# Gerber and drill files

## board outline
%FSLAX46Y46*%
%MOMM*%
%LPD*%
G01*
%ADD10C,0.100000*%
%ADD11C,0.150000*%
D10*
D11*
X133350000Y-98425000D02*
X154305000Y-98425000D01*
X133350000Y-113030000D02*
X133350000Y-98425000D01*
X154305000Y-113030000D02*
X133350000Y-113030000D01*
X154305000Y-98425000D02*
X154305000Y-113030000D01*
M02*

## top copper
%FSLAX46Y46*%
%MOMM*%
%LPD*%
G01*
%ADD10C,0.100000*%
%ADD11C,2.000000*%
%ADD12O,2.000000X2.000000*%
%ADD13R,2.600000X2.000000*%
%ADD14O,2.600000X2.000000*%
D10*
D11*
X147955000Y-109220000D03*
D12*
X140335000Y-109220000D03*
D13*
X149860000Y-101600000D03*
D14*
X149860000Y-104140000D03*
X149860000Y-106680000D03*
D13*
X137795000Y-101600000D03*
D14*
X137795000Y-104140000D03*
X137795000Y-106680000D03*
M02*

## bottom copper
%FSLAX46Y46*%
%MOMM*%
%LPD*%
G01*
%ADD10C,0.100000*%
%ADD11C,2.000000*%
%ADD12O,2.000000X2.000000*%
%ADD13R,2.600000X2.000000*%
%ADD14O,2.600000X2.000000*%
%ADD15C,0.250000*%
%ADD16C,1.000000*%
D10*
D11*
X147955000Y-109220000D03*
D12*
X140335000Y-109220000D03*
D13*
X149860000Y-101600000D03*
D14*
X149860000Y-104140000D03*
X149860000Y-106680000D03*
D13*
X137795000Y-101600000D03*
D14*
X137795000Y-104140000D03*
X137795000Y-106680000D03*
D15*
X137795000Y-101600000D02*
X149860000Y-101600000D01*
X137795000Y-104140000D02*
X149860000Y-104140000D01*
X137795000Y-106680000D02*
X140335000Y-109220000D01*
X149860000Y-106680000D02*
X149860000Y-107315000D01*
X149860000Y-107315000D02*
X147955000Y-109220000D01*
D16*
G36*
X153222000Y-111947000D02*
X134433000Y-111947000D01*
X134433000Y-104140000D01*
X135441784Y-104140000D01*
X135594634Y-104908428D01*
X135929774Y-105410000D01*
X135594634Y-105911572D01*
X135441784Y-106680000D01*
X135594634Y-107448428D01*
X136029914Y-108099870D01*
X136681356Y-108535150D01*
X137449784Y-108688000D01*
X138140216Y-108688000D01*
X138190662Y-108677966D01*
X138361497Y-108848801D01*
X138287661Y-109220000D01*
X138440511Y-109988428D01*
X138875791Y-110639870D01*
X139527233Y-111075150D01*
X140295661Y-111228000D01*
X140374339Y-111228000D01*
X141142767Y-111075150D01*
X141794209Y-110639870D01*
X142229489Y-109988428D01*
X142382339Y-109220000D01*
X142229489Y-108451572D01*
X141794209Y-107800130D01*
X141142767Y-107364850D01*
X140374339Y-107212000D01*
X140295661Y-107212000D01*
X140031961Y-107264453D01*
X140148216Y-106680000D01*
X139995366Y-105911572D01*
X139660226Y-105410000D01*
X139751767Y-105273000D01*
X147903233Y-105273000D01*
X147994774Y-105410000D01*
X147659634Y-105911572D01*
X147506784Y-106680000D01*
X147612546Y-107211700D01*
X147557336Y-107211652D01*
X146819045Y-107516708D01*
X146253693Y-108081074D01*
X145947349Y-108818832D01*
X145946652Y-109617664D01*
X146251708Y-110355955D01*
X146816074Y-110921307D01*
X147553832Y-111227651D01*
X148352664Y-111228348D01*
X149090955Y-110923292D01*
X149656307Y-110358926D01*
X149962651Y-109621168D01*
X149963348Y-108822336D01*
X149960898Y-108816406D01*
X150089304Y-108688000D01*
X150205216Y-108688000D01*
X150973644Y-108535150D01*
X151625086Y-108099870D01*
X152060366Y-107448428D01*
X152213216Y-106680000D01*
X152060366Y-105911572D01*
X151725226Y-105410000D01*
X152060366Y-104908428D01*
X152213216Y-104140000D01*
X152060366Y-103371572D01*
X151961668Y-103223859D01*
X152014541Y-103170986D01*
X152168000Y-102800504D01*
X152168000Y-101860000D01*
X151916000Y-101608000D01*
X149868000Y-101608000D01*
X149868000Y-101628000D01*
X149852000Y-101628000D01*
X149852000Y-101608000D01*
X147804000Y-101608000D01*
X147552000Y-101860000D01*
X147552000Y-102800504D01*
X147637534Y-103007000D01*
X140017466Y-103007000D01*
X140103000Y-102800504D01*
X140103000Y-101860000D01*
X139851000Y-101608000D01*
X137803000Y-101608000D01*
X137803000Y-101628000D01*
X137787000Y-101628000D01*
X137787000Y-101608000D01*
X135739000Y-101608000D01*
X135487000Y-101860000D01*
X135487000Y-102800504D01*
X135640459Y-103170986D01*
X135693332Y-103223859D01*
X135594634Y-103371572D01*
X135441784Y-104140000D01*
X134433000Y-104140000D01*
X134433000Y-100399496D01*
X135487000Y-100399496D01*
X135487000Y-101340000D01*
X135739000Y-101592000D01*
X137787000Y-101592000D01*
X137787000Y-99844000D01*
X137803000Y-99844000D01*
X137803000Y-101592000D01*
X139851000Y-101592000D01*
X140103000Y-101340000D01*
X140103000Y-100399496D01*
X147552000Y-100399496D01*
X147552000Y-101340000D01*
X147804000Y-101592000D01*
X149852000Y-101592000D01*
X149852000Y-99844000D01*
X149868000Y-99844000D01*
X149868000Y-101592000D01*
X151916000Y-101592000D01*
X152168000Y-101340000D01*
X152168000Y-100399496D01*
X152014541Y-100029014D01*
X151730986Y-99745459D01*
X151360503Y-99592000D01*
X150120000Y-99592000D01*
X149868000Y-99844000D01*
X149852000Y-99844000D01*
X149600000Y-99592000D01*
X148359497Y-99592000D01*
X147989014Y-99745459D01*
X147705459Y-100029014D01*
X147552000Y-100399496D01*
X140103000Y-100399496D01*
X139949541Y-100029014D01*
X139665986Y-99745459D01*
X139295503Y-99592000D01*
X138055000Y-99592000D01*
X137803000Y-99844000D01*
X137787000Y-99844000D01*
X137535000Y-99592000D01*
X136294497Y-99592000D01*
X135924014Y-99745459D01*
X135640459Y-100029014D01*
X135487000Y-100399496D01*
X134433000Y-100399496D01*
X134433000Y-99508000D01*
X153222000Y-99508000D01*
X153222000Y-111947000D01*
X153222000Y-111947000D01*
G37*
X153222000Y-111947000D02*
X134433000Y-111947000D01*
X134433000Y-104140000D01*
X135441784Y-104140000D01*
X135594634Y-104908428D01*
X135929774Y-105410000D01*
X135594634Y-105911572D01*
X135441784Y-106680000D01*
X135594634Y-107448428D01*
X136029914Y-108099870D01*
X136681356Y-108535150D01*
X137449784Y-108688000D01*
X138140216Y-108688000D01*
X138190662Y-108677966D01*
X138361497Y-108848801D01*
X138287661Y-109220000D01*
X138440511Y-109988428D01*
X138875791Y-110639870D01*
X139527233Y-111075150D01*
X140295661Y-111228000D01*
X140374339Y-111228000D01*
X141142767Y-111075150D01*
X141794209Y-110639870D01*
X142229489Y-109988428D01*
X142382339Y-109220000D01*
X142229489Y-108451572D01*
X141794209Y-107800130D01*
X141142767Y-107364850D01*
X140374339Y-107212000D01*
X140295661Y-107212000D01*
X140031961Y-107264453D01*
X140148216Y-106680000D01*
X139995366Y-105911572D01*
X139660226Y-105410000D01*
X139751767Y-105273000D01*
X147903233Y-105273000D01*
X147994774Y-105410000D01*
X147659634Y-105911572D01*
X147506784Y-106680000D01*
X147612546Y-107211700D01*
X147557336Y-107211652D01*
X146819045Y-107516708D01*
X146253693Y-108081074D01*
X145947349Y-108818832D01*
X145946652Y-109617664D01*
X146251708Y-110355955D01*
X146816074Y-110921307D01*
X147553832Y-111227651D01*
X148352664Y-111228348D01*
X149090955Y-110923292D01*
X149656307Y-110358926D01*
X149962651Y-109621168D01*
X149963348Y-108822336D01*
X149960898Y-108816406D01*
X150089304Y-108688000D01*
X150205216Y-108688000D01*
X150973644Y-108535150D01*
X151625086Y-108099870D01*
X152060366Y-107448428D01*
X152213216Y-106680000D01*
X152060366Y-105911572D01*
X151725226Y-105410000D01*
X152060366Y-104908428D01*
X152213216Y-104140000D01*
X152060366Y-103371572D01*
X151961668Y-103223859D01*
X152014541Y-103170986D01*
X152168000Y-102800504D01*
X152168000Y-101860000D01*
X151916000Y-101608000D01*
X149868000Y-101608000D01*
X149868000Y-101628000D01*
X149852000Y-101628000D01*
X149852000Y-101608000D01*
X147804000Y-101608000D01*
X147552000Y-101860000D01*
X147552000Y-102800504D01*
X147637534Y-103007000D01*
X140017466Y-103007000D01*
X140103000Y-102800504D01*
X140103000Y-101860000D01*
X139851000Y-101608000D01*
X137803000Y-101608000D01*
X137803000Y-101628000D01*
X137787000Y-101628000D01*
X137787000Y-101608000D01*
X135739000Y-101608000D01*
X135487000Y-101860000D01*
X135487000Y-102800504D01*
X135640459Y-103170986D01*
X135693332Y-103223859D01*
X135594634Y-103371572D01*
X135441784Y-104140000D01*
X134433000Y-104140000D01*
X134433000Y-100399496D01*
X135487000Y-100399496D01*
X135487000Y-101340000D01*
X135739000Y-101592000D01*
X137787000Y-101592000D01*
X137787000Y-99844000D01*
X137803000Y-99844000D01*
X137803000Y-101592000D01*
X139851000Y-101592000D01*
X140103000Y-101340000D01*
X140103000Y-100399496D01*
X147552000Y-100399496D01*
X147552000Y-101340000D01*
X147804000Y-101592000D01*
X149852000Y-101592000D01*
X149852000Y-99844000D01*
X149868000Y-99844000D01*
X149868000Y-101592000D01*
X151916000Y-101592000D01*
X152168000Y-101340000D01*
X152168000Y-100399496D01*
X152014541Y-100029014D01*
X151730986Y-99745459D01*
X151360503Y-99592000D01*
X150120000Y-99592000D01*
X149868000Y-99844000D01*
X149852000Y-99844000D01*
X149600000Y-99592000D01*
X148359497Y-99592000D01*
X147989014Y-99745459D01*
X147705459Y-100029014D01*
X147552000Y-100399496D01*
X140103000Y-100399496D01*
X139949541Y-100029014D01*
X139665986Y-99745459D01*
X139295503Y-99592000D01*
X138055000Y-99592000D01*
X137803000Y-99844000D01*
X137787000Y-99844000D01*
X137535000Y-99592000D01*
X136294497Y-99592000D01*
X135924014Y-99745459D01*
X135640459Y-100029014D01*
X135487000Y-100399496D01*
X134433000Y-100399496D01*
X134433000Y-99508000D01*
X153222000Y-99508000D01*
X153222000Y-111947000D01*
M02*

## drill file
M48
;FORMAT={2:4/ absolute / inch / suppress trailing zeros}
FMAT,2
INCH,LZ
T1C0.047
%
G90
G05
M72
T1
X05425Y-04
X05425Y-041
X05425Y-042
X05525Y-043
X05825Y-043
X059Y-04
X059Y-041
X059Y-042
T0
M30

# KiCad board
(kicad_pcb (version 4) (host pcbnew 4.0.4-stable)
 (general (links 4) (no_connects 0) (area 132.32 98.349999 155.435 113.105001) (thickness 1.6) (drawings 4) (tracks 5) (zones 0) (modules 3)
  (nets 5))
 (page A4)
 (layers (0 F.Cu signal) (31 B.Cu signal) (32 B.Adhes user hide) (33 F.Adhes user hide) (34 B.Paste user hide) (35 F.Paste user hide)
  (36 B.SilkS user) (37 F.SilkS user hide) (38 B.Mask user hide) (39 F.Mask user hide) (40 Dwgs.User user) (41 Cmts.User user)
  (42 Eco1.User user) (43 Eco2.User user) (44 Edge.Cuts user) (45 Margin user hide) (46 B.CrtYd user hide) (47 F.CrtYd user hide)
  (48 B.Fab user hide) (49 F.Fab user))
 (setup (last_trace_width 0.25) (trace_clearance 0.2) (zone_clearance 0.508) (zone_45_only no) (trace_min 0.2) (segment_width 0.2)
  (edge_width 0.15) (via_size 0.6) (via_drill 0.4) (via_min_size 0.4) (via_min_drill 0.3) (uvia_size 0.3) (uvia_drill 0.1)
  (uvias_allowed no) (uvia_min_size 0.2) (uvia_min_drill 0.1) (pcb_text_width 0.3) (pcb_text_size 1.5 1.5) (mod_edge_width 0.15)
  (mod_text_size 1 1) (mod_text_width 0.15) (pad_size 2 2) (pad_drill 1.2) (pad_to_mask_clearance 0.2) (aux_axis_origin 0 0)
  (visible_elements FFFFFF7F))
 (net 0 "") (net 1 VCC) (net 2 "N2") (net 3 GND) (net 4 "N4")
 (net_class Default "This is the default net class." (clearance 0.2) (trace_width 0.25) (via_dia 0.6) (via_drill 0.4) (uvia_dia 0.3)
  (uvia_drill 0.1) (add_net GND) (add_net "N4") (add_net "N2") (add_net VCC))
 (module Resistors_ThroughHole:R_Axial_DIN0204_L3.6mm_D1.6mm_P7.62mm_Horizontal (layer F.Cu) (at 147.955 109.22 180)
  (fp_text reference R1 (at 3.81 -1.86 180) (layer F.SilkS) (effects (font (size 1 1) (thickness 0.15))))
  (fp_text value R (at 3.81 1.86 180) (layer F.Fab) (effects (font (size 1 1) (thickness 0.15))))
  (pad 1 thru_hole circle (at 0 0 180) (size 2 2) (drill 1.2) (layers *.Cu *.Mask) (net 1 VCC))
  (pad 2 thru_hole oval (at 7.62 0 180) (size 2 2) (drill 1.2) (layers *.Cu *.Mask) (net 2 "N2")))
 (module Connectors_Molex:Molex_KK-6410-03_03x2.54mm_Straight (layer F.Cu) (at 149.86 101.6 270)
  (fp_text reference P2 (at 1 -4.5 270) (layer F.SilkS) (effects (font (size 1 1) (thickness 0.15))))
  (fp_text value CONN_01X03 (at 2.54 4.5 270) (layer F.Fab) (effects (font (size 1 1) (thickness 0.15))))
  (pad 1 thru_hole rect (at 0 0 270) (size 2 2.6) (drill 1.2) (layers *.Cu *.Mask) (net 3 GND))
  (pad 2 thru_hole oval (at 2.54 0 270) (size 2 2.6) (drill 1.2) (layers *.Cu *.Mask) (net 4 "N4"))
  (pad 3 thru_hole oval (at 5.08 0 270) (size 2 2.6) (drill 1.2) (layers *.Cu *.Mask) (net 1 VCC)))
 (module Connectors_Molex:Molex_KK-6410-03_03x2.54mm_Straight (layer F.Cu) (at 137.795 101.6 270)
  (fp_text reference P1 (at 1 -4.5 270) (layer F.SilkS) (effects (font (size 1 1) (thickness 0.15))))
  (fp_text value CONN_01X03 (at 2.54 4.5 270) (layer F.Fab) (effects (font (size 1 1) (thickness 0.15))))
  (pad 1 thru_hole rect (at 0 0 270) (size 2 2.6) (drill 1.2) (layers *.Cu *.Mask) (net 3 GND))
  (pad 2 thru_hole oval (at 2.54 0 270) (size 2 2.6) (drill 1.2) (layers *.Cu *.Mask) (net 4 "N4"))
  (pad 3 thru_hole oval (at 5.08 0 270) (size 2 2.6) (drill 1.2) (layers *.Cu *.Mask) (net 2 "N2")))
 (gr_line (start 133.35 98.425) (end 154.305 98.425) (angle 90) (layer Edge.Cuts) (width 0.15))
 (gr_line (start 133.35 113.03) (end 133.35 98.425) (angle 90) (layer Edge.Cuts) (width 0.15))
 (gr_line (start 154.305 113.03) (end 133.35 113.03) (angle 90) (layer Edge.Cuts) (width 0.15))
 (gr_line (start 154.305 98.425) (end 154.305 113.03) (angle 90) (layer Edge.Cuts) (width 0.15))
 (segment (start 137.795 101.6) (end 149.86 101.6) (width 0.25) (layer B.Cu) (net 3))
 (segment (start 137.795 104.14) (end 149.86 104.14) (width 0.25) (layer B.Cu) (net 4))
 (segment (start 137.795 106.68) (end 140.335 109.22) (width 0.25) (layer B.Cu) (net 2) (status C00000))
 (segment (start 149.86 106.68) (end 149.86 107.315) (width 0.25) (layer B.Cu) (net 1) (status C00000))
 (segment (start 149.86 107.315) (end 147.955 109.22) (width 0.25) (layer B.Cu) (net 1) (status C00000))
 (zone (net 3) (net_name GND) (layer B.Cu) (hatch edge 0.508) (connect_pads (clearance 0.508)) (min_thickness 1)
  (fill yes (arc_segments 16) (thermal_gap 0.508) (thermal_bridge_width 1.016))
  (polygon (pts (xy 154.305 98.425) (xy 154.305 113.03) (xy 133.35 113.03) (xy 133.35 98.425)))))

